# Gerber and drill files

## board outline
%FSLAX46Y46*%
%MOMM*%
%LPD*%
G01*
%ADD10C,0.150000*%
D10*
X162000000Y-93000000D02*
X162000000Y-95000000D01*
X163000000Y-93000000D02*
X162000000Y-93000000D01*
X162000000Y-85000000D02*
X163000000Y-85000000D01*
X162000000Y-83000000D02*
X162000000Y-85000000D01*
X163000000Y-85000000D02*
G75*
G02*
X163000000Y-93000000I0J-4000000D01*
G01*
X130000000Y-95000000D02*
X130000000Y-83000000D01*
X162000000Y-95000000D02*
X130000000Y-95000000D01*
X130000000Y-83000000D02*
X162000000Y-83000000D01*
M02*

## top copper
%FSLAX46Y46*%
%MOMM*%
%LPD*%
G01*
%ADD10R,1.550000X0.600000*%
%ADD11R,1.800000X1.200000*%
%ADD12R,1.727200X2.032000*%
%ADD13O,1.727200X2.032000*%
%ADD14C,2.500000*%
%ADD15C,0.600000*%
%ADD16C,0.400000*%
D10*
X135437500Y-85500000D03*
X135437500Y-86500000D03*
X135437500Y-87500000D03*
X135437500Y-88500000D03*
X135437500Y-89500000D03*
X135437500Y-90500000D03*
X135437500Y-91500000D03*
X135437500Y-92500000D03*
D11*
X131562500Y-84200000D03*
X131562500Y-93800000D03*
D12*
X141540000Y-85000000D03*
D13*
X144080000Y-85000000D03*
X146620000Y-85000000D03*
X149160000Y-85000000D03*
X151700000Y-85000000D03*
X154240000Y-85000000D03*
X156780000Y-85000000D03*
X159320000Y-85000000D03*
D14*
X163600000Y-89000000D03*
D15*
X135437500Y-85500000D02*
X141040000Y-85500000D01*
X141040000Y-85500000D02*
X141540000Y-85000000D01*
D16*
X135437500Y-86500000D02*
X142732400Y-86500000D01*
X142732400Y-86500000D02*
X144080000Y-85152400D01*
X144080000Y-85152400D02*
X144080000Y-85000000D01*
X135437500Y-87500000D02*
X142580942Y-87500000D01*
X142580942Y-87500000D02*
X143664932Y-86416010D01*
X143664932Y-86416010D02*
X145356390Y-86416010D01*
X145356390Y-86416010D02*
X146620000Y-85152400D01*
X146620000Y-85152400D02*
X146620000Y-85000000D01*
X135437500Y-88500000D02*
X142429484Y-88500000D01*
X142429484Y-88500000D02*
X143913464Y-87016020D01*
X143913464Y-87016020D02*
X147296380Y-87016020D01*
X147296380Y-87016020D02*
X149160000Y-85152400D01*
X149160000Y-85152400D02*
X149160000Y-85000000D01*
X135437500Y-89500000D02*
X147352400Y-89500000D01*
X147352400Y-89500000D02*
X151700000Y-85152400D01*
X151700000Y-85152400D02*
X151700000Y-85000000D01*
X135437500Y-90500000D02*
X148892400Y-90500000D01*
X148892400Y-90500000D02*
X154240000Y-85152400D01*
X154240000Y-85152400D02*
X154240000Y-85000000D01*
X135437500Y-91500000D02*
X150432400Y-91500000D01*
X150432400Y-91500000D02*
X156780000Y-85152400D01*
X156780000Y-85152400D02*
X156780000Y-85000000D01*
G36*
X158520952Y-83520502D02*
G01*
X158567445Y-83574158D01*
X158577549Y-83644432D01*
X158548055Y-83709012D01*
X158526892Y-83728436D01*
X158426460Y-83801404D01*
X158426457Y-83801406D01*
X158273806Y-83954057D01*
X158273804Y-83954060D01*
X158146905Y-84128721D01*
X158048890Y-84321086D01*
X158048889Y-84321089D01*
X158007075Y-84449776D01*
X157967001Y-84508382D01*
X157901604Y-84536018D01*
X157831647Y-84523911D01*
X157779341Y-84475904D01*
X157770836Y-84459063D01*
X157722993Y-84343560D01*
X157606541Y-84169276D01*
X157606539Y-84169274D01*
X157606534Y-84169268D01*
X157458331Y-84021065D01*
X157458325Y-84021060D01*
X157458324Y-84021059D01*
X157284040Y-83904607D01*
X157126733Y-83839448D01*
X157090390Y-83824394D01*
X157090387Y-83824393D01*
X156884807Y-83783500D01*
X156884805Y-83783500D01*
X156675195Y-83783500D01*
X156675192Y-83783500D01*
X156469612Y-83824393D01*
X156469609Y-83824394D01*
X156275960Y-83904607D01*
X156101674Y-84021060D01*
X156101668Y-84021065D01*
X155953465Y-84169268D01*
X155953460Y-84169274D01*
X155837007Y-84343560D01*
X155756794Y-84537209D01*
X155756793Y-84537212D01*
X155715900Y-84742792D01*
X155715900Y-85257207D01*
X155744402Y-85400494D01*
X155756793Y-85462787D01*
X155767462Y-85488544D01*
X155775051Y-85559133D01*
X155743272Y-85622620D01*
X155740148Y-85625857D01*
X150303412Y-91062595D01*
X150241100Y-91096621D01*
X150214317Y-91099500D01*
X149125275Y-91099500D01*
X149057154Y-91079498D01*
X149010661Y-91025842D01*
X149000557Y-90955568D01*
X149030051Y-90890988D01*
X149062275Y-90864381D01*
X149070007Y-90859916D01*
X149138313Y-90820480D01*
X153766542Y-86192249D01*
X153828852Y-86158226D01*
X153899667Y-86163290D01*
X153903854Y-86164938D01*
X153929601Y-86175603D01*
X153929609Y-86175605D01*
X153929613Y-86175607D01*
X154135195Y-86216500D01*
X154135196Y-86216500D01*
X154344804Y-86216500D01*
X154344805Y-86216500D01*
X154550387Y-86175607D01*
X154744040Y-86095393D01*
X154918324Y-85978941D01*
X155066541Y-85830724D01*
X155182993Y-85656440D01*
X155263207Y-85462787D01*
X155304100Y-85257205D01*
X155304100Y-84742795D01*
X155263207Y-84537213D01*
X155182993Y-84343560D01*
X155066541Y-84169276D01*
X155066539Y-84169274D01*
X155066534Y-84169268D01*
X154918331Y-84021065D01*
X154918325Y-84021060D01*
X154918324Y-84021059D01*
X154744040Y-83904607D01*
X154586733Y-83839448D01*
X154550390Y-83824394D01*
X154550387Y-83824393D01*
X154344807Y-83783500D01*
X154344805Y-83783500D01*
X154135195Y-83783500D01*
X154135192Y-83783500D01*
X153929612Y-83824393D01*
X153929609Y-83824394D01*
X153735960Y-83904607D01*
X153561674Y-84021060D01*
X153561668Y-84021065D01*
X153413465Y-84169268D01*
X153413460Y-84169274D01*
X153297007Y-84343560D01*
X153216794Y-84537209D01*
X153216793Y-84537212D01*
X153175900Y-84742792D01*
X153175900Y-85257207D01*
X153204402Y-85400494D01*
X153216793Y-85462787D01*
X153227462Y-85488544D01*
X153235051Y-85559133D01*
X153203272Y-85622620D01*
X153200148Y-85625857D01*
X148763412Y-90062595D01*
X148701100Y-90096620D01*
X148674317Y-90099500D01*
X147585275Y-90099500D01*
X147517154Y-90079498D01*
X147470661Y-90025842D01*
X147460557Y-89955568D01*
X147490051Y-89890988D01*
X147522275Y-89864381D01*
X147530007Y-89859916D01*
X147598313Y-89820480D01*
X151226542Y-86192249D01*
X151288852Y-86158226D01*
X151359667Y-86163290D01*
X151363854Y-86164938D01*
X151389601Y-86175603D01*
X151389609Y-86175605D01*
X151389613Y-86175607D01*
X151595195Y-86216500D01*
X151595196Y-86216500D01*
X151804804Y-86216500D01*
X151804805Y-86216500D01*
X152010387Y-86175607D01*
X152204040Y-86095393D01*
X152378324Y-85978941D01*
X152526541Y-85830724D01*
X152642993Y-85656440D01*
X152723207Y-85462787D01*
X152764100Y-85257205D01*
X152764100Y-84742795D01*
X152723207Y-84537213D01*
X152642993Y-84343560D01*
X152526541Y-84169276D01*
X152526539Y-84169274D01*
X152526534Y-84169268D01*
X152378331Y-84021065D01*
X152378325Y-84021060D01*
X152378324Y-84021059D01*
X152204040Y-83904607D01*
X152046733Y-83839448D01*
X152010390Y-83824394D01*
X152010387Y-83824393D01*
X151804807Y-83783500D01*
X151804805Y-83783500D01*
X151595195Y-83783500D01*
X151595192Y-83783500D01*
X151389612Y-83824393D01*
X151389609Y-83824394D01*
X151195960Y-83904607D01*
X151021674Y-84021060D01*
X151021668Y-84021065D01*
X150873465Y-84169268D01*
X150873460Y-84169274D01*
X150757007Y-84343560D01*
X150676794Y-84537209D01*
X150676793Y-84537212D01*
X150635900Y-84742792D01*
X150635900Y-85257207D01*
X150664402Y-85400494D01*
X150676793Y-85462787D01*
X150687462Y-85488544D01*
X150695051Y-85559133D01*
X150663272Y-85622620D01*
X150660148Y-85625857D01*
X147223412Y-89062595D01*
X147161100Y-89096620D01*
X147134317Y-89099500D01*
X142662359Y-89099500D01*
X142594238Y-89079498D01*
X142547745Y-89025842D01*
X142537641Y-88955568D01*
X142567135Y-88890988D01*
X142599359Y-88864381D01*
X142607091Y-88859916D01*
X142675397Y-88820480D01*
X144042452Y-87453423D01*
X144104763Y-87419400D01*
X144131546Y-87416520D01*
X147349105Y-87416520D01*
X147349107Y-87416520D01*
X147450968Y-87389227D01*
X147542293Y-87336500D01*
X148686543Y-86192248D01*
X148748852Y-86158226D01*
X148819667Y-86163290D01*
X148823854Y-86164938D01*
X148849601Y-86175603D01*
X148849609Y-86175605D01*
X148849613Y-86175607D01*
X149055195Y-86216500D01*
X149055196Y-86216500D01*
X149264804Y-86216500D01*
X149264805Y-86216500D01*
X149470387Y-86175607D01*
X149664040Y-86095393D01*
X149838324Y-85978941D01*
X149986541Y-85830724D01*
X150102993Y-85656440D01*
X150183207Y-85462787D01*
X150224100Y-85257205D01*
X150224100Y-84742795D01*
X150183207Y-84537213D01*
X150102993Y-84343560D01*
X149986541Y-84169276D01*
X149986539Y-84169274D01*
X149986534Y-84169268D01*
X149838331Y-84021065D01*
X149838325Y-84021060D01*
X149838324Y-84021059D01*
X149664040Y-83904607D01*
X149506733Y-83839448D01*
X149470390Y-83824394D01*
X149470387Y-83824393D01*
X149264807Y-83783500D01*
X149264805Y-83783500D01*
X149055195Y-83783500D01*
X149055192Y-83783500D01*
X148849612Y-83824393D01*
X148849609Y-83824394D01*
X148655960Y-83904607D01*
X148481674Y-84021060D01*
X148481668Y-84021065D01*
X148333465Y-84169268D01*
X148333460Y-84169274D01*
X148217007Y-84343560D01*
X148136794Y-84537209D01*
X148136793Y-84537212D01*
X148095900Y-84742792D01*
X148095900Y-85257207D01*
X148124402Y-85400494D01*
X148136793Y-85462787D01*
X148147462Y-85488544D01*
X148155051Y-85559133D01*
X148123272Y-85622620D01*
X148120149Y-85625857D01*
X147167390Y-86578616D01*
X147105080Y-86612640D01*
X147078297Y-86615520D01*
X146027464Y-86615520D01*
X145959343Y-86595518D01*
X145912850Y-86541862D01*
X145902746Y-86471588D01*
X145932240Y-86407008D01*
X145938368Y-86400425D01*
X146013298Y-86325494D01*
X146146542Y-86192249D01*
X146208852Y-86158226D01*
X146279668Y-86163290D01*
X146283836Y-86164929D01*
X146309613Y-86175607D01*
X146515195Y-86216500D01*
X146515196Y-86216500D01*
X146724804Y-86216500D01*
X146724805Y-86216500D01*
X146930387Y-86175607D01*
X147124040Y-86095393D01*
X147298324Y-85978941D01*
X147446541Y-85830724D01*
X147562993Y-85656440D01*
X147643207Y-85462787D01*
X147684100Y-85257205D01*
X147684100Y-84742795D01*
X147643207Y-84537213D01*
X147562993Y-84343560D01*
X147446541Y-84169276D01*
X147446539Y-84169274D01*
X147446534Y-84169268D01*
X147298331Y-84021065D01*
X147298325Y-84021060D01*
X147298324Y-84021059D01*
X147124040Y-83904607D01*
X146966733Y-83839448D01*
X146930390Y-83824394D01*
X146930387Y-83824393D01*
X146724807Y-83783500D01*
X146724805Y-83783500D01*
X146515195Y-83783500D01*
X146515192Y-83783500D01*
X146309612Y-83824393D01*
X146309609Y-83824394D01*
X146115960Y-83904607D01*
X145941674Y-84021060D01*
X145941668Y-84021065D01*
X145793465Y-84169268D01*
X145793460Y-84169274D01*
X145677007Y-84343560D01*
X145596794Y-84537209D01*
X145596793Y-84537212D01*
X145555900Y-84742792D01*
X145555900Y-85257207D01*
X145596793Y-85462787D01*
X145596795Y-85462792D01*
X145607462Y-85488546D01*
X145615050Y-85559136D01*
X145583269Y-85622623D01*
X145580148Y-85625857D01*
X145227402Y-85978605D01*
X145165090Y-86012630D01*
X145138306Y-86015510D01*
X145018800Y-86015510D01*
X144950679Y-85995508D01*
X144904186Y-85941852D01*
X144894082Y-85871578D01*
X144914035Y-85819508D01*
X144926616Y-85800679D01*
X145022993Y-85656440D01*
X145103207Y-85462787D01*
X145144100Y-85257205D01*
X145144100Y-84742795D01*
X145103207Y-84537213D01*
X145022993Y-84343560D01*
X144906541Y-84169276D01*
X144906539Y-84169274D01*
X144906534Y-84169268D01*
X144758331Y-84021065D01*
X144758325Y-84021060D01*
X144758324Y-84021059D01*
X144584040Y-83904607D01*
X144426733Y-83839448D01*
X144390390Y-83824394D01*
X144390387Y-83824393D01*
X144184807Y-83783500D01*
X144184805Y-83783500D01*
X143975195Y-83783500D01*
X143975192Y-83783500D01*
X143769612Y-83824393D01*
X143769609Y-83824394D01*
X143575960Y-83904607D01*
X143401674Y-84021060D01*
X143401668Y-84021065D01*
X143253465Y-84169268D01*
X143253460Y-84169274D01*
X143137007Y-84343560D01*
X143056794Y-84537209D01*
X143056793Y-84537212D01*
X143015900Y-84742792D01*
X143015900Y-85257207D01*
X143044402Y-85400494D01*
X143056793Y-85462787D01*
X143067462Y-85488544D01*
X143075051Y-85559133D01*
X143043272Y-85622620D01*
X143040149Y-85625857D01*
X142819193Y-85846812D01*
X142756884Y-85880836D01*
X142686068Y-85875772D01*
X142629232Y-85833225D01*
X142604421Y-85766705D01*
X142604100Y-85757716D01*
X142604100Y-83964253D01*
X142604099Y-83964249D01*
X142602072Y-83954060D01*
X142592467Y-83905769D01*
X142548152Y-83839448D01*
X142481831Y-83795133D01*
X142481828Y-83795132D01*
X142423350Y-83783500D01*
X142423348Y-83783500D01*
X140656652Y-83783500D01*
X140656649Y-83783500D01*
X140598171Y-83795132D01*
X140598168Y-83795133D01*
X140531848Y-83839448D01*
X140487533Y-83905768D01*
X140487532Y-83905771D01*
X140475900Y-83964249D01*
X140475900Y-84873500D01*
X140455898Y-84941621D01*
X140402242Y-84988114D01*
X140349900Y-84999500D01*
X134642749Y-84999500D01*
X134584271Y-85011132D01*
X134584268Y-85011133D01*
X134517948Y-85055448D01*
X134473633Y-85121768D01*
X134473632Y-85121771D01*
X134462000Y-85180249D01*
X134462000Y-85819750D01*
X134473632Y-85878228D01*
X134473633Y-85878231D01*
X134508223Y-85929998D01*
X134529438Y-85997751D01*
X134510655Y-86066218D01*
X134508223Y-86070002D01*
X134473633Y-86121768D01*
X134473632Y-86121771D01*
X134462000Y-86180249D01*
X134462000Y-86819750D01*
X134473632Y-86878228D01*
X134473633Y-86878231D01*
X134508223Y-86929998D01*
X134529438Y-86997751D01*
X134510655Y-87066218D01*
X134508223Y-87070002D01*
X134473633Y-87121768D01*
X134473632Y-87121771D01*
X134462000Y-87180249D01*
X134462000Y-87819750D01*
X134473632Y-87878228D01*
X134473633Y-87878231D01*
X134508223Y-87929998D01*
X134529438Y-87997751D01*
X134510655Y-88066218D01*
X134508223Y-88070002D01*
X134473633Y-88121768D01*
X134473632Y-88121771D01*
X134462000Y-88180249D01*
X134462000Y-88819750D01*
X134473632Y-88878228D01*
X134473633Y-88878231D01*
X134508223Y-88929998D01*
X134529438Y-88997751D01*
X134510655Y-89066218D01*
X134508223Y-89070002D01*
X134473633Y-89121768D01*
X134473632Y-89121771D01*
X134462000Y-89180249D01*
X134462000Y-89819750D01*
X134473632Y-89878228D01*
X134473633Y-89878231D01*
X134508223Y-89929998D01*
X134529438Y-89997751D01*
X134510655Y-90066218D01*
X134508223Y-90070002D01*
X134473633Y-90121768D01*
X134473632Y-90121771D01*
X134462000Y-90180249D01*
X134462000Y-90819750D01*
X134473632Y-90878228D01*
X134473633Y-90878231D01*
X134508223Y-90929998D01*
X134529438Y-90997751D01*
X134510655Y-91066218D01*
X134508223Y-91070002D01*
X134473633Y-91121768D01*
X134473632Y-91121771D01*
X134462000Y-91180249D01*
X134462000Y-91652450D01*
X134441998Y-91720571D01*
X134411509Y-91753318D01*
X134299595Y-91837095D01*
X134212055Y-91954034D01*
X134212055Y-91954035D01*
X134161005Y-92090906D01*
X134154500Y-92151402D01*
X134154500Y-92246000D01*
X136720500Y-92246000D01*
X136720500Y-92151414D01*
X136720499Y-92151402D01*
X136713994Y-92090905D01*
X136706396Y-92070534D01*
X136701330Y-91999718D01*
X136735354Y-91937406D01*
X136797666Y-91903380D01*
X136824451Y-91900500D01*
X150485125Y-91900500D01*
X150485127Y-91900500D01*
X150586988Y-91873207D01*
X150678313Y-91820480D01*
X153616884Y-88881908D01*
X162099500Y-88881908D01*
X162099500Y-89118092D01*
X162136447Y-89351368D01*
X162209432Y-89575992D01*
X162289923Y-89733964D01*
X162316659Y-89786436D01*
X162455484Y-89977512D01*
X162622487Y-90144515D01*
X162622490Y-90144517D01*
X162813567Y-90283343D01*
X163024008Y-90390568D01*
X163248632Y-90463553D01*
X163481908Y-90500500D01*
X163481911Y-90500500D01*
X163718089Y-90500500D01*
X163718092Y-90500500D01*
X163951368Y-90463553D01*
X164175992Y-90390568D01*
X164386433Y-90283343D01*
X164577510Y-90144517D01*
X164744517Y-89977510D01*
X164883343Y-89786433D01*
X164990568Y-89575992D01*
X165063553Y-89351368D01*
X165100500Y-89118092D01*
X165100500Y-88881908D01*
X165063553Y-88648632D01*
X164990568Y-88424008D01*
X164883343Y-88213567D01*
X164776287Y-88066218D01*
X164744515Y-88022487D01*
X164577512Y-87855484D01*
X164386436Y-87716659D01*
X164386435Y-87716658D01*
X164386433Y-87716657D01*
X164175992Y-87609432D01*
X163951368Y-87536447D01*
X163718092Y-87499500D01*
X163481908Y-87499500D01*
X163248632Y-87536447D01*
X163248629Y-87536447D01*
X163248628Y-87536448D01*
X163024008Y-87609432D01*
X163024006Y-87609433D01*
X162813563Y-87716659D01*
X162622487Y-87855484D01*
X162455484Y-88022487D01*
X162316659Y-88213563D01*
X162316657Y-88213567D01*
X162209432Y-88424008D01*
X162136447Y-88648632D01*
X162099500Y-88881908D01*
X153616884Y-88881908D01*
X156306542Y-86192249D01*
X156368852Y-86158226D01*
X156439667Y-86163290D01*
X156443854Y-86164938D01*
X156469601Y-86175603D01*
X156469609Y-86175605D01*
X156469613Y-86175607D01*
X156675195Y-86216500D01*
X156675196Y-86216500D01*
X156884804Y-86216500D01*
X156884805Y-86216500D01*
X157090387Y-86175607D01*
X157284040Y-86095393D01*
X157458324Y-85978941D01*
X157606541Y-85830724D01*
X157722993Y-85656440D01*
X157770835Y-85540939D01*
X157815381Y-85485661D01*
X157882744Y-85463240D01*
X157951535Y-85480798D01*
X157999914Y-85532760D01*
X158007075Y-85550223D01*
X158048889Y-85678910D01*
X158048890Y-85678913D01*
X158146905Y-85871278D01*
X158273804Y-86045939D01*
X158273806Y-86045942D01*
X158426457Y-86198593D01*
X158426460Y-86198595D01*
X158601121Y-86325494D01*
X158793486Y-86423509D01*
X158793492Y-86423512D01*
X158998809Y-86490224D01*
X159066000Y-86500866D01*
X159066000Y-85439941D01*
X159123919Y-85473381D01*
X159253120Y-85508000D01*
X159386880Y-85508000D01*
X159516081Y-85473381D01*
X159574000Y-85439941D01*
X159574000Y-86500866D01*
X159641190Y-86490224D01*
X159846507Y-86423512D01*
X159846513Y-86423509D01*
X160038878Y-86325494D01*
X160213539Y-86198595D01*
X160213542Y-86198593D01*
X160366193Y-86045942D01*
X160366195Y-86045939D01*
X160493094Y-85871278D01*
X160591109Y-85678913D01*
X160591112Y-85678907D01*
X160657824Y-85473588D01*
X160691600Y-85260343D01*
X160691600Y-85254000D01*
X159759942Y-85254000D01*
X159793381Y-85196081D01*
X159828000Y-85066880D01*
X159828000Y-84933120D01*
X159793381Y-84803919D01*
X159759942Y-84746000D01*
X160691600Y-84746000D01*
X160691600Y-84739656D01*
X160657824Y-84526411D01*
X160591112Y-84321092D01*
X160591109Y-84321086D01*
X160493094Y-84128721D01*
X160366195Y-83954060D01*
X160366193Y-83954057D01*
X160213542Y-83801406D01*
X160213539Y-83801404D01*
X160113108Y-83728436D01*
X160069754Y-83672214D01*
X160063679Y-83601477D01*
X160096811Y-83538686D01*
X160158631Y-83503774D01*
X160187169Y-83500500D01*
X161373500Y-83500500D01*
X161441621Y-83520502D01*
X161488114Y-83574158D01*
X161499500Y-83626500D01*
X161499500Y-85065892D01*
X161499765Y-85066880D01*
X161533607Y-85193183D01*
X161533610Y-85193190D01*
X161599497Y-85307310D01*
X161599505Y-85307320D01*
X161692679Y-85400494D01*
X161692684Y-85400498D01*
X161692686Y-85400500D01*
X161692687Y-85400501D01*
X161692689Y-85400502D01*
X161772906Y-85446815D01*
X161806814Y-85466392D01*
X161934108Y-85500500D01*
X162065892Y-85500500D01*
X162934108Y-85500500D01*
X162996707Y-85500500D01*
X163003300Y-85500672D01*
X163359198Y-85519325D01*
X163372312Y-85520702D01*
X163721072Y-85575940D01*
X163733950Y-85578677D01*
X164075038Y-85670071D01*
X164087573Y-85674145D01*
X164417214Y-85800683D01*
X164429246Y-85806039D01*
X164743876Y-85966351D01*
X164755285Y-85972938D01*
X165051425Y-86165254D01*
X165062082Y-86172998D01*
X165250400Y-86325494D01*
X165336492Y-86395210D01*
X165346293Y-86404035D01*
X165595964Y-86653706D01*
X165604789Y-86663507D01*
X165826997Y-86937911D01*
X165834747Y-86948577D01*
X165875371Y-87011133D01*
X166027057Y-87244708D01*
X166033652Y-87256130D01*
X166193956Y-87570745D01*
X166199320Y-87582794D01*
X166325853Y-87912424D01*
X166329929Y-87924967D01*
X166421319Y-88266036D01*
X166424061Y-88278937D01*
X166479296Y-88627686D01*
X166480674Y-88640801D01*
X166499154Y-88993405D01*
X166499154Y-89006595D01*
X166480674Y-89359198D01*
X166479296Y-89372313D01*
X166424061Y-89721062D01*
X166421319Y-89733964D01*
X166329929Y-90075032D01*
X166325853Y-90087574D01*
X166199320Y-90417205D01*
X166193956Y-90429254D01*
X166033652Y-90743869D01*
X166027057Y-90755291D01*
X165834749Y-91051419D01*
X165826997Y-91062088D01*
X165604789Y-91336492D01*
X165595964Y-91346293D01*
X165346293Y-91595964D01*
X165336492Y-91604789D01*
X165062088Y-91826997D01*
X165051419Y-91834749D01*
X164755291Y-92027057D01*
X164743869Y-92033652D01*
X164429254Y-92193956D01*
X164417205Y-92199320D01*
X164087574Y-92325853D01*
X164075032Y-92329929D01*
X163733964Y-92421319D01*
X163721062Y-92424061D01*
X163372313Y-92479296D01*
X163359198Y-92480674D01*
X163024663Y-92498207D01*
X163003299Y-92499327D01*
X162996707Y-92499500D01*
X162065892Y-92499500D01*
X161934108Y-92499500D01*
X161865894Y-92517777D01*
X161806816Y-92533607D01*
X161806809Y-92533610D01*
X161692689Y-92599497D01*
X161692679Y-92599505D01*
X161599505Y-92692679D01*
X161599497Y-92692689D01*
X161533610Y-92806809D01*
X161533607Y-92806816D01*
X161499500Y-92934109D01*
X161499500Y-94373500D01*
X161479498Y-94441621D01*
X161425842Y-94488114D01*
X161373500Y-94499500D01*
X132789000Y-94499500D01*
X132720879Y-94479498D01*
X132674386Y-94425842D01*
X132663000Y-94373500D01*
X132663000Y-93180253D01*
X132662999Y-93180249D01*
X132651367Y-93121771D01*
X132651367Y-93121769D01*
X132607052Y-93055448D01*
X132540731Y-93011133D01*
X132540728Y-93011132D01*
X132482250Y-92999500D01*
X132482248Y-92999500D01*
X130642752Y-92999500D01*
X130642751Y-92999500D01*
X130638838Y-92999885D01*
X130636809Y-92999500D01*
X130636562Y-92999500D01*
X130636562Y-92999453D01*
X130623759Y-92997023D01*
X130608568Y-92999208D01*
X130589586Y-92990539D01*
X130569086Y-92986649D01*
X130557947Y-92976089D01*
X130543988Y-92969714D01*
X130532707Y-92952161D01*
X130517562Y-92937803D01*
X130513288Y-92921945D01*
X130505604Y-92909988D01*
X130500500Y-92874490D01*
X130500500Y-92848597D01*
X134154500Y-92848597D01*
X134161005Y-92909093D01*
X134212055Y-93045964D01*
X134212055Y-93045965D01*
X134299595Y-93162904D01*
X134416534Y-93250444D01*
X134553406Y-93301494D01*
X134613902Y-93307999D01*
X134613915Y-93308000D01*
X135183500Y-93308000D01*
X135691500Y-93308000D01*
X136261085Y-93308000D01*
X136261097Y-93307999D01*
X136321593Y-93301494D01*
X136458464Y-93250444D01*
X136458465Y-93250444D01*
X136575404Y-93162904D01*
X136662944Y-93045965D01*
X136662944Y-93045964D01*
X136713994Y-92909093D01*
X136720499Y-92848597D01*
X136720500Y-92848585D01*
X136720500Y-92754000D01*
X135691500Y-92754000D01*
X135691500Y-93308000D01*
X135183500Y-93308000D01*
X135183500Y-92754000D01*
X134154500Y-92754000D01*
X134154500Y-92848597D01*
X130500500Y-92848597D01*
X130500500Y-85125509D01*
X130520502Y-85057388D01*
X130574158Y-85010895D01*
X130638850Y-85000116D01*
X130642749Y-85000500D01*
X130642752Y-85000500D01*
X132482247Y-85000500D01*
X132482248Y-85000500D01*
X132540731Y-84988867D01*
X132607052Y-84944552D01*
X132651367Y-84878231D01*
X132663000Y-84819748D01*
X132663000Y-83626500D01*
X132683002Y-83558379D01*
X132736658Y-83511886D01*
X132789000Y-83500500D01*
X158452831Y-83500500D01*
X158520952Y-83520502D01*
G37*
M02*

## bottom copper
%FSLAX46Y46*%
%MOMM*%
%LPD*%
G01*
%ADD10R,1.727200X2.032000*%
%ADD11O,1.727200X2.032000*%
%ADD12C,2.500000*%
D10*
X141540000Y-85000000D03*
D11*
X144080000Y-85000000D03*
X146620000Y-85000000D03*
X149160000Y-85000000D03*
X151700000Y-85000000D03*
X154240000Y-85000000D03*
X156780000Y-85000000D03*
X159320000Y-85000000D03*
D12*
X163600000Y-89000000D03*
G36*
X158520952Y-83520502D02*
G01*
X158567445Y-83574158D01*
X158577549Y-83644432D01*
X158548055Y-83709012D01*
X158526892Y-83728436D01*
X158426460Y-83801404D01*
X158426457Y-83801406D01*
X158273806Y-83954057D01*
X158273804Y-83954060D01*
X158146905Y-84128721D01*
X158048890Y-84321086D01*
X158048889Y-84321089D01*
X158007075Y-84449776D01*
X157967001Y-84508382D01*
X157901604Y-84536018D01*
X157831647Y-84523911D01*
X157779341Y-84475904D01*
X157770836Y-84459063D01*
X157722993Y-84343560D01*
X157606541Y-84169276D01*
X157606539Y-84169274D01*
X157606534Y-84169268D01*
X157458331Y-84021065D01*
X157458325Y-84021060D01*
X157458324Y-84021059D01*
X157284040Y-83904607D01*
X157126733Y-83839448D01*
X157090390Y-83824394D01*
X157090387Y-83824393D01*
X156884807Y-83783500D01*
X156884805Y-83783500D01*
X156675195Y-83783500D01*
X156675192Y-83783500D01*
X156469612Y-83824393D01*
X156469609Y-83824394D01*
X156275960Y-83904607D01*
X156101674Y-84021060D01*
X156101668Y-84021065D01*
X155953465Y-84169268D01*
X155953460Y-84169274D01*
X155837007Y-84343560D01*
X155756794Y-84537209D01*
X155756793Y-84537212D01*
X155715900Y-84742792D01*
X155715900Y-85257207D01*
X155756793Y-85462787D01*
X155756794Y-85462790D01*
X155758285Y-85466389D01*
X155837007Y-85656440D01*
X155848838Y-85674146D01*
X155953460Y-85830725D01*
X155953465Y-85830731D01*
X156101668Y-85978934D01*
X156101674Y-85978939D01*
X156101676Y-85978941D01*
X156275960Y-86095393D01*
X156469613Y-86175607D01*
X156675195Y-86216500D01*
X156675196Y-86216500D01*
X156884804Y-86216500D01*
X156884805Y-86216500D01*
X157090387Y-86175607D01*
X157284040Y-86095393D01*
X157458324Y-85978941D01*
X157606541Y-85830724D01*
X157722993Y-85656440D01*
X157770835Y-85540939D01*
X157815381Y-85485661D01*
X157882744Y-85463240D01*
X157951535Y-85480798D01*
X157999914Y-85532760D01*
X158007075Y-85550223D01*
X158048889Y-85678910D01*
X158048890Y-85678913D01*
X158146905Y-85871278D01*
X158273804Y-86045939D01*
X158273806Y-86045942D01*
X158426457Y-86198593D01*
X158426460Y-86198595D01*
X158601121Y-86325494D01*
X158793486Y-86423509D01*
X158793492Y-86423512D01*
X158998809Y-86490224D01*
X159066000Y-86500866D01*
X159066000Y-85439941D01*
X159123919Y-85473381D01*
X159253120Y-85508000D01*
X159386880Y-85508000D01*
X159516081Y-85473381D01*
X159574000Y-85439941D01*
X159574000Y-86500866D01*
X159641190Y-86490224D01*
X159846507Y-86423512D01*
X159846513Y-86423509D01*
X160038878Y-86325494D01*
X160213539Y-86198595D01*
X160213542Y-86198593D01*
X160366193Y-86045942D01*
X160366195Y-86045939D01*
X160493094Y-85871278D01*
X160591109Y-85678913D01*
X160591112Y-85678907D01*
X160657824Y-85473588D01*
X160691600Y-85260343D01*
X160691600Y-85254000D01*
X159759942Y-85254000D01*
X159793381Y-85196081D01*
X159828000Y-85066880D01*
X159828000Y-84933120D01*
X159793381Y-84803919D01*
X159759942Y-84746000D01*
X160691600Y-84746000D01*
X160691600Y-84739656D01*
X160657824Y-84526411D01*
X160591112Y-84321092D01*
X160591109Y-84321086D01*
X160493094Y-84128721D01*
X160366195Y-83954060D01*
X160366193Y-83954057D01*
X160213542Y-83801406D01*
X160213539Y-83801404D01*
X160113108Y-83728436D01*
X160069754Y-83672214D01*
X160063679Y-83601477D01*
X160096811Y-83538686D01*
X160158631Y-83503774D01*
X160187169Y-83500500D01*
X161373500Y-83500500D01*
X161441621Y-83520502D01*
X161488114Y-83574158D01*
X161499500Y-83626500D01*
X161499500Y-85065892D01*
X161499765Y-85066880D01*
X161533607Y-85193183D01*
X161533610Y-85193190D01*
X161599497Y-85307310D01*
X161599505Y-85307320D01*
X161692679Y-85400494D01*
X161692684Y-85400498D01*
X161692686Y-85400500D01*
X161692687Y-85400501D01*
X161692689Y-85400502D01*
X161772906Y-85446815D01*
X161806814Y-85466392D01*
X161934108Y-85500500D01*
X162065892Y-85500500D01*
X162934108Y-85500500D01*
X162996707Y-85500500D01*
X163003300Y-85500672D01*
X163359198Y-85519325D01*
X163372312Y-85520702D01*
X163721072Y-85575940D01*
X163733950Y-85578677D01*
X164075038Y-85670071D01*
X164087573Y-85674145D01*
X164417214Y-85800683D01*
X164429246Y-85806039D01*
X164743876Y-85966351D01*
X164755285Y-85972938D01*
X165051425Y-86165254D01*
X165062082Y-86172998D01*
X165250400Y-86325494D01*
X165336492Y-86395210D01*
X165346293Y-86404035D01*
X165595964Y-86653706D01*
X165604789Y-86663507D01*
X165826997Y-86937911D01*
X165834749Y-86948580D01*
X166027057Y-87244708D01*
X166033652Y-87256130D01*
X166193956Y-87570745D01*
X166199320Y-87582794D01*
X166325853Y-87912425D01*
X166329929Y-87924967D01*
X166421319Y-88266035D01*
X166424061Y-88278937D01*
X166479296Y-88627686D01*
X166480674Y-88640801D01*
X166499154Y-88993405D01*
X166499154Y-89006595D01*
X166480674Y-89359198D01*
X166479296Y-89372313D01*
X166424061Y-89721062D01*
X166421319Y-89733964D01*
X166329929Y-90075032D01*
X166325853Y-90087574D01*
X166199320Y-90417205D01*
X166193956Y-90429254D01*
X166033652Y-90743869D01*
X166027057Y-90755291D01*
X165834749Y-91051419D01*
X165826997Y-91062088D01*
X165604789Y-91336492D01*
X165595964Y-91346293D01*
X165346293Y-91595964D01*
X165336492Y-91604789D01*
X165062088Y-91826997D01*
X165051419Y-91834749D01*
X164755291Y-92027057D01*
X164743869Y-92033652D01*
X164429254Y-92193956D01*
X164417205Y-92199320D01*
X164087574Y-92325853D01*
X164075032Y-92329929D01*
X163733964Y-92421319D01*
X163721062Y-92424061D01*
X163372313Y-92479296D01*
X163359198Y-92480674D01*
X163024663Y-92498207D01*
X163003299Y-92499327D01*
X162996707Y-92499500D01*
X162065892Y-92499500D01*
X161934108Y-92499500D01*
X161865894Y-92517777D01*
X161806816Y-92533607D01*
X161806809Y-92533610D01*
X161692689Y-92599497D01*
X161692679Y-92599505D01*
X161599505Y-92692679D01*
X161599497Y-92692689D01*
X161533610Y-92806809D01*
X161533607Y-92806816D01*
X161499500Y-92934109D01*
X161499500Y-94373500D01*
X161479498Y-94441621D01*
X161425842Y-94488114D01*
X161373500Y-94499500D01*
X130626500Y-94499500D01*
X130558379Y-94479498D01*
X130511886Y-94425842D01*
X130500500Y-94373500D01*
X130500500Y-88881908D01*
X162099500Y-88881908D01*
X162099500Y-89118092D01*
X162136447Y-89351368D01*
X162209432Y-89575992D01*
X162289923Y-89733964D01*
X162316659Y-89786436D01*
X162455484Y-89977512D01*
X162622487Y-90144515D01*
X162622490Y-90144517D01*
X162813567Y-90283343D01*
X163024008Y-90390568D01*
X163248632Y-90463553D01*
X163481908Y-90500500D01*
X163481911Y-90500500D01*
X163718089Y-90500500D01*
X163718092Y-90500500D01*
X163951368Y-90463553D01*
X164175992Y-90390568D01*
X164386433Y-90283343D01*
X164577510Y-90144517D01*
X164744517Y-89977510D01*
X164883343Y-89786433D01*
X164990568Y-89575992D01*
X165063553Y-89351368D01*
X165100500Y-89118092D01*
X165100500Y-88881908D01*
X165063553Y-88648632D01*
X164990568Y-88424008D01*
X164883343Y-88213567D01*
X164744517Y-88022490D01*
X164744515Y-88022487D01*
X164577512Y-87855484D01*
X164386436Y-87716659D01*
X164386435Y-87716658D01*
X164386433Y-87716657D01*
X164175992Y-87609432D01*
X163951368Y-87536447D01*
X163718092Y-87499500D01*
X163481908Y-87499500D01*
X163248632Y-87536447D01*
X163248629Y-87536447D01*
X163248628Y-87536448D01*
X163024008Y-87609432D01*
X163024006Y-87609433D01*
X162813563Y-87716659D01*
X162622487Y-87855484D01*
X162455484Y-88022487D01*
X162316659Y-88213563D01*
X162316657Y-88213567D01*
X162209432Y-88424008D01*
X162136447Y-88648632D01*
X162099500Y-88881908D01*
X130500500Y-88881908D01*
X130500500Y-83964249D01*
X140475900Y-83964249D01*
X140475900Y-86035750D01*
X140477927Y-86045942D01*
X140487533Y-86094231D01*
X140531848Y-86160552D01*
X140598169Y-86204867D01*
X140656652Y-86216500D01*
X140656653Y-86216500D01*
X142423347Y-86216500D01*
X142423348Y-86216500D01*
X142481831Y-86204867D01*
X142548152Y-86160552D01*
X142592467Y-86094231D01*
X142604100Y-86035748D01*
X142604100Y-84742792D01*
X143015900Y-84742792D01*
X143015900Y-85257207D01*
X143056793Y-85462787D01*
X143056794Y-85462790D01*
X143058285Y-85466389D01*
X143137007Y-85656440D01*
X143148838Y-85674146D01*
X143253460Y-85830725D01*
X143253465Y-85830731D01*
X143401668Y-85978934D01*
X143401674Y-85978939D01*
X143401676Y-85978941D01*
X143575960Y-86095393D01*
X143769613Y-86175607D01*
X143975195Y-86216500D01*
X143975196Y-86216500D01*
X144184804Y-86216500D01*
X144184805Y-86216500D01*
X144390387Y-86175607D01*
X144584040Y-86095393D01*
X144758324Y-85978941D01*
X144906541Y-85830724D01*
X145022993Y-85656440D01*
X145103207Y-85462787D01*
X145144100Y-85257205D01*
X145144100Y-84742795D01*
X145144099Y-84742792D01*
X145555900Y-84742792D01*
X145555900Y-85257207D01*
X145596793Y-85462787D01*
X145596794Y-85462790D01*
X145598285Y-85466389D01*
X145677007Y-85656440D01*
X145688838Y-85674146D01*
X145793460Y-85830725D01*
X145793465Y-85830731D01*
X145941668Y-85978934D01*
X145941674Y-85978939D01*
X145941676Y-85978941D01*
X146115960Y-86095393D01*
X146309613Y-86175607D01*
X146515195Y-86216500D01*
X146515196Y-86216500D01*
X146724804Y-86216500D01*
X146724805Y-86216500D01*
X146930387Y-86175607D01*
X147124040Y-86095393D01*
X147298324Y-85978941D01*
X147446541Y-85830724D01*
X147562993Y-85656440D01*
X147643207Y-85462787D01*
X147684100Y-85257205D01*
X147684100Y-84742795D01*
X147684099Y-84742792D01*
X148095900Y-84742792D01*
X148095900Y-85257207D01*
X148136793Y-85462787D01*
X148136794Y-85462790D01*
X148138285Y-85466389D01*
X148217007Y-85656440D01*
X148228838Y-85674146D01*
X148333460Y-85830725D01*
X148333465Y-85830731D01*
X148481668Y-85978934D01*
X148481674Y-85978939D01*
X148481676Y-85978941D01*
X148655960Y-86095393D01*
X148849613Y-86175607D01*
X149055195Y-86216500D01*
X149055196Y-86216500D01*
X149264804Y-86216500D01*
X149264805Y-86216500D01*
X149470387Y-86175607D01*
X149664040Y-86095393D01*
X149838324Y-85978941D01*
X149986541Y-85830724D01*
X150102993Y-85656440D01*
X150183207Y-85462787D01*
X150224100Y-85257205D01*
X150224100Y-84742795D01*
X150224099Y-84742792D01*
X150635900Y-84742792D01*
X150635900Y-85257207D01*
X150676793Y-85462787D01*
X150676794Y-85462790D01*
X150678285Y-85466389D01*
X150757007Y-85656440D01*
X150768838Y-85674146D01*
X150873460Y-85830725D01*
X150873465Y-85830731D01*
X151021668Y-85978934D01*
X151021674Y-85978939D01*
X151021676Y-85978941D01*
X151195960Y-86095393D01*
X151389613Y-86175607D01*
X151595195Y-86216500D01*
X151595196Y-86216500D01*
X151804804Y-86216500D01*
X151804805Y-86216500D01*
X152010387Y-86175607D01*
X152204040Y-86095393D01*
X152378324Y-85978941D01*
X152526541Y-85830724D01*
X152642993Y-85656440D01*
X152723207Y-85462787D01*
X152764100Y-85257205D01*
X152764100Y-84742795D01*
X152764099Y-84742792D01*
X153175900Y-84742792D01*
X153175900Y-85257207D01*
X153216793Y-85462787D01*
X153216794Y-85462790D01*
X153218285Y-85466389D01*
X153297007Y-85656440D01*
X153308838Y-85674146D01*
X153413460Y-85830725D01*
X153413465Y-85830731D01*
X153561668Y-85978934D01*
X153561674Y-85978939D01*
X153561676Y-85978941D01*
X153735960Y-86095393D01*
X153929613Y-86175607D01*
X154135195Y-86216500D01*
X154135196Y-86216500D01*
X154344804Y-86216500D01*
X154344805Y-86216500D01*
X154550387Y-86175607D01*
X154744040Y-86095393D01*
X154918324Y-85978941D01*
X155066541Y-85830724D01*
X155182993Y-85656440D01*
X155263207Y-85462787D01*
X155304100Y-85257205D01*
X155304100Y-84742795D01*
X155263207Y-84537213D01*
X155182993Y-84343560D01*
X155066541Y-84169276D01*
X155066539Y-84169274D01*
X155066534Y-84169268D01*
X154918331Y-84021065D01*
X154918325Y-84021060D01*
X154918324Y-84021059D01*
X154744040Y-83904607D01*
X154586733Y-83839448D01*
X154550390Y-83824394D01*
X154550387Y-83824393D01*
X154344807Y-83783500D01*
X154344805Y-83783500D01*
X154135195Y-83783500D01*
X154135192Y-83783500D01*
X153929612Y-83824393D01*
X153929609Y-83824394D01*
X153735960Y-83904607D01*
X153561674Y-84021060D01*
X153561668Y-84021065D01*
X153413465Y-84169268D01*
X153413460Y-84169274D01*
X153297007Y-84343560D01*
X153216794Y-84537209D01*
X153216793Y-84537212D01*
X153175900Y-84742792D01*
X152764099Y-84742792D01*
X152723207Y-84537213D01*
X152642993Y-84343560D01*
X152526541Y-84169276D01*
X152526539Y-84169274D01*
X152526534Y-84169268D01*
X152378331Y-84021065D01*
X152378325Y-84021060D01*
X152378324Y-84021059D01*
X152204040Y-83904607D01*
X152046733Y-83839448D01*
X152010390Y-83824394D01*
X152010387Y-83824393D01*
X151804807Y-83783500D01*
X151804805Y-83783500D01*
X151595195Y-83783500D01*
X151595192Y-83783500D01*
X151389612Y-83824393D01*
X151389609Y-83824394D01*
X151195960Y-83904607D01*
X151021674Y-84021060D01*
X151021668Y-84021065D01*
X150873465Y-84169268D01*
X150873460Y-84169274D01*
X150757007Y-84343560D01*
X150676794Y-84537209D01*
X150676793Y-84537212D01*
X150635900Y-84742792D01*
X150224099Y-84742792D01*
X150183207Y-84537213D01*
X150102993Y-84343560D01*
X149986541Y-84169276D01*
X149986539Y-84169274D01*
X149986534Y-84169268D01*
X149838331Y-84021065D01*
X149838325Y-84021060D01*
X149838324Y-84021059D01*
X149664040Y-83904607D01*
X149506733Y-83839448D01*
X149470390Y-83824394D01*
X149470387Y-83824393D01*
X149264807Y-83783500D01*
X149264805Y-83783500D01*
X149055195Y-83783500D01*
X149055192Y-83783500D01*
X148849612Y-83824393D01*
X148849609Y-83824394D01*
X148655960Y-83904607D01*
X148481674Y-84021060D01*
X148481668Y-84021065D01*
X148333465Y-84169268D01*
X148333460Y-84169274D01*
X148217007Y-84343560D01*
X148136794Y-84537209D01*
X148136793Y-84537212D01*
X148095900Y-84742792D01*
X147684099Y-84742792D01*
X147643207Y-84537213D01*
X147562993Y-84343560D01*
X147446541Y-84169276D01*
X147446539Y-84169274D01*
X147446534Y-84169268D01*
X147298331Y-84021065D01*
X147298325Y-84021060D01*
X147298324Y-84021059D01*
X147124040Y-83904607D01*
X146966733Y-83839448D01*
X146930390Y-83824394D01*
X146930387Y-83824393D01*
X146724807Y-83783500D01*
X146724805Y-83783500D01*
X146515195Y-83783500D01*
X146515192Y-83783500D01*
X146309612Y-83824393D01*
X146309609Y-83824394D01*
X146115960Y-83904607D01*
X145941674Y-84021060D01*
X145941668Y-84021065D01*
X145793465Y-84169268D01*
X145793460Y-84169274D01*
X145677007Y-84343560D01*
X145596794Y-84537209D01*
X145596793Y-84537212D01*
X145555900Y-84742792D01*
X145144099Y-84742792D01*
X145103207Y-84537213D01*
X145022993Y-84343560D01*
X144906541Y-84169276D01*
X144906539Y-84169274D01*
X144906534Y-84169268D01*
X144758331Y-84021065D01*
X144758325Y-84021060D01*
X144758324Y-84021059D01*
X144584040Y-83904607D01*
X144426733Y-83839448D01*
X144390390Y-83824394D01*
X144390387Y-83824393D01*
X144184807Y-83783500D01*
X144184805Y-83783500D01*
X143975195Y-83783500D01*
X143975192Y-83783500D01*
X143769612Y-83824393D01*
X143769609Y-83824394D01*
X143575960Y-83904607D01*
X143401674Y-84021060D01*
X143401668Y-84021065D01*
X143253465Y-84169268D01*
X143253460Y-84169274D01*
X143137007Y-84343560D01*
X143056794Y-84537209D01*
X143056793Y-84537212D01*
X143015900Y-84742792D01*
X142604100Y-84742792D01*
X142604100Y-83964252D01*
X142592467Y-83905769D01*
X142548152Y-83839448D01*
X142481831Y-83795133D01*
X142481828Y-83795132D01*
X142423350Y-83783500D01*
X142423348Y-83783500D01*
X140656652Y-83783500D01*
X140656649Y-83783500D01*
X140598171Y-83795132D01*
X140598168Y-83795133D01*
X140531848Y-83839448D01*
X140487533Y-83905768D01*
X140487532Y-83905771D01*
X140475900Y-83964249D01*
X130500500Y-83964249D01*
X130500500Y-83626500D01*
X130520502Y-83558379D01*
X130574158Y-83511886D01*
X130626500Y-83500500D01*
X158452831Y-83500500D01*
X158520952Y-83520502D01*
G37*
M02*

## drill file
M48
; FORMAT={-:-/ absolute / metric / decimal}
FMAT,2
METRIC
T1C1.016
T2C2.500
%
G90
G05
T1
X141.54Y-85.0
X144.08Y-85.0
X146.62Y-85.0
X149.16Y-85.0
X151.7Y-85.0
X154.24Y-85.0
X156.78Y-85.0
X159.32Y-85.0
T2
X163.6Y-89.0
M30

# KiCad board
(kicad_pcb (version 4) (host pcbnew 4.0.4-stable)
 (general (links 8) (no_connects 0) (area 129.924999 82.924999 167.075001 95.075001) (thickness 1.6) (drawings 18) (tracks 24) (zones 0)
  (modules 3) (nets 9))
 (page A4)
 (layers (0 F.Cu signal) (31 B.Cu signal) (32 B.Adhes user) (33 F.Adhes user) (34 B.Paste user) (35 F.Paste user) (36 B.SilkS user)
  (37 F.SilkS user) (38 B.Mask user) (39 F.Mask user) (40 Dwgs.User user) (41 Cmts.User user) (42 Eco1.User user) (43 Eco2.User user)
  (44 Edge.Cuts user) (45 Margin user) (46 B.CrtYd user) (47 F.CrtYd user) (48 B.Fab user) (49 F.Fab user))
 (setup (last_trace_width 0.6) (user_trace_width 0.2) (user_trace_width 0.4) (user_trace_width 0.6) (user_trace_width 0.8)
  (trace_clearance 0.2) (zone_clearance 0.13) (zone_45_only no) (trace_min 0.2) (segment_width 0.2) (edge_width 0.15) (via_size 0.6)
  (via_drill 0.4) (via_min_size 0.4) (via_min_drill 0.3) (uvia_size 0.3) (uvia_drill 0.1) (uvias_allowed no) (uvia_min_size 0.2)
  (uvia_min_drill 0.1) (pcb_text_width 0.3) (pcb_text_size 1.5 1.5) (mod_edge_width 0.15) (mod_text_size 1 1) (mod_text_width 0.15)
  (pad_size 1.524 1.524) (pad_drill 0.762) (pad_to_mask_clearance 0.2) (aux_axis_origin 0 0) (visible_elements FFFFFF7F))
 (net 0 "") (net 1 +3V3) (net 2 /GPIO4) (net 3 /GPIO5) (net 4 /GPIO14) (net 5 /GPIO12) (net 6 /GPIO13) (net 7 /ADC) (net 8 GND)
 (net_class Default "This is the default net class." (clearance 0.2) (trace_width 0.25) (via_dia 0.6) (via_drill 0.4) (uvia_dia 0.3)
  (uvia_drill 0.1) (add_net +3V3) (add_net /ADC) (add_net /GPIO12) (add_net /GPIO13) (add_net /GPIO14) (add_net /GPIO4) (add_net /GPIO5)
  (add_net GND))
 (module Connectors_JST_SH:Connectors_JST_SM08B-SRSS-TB (layer F.Cu) (at 133.5 89 270)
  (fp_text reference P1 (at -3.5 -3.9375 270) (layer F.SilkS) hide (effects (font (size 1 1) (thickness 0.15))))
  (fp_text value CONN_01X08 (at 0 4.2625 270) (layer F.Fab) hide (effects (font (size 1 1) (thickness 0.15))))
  (pad 1 smd rect (at -3.5 -1.9375 270) (size 0.6 1.55) (layers F.Cu F.Paste F.Mask) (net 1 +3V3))
  (pad 2 smd rect (at -2.5 -1.9375 270) (size 0.6 1.55) (layers F.Cu F.Paste F.Mask) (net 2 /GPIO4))
  (pad 3 smd rect (at -1.5 -1.9375 270) (size 0.6 1.55) (layers F.Cu F.Paste F.Mask) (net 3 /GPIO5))
  (pad 4 smd rect (at -0.5 -1.9375 270) (size 0.6 1.55) (layers F.Cu F.Paste F.Mask) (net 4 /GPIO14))
  (pad 5 smd rect (at 0.5 -1.9375 270) (size 0.6 1.55) (layers F.Cu F.Paste F.Mask) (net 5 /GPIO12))
  (pad 6 smd rect (at 1.5 -1.9375 270) (size 0.6 1.55) (layers F.Cu F.Paste F.Mask) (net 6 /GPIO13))
  (pad 7 smd rect (at 2.5 -1.9375 270) (size 0.6 1.55) (layers F.Cu F.Paste F.Mask) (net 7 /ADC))
  (pad 8 smd rect (at 3.5 -1.9375 270) (size 0.6 1.55) (layers F.Cu F.Paste F.Mask) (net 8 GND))
  (pad "" smd rect (at -4.8 1.9375 270) (size 1.2 1.8) (layers F.Cu F.Paste F.Mask))
  (pad "" smd rect (at 4.8 1.9375 270) (size 1.2 1.8) (layers F.Cu F.Paste F.Mask)))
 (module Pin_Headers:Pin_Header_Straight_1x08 (layer F.Cu) (at 141.54 85 90)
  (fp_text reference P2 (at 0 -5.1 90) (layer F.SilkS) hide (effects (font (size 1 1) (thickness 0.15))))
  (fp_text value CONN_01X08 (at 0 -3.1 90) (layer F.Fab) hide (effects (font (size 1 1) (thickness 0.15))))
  (pad 1 thru_hole rect (at 0 0 90) (size 2.032 1.7272) (drill 1.016) (layers *.Cu *.Mask F.SilkS) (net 1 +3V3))
  (pad 2 thru_hole oval (at 0 2.54 90) (size 2.032 1.7272) (drill 1.016) (layers *.Cu *.Mask F.SilkS) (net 2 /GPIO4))
  (pad 3 thru_hole oval (at 0 5.08 90) (size 2.032 1.7272) (drill 1.016) (layers *.Cu *.Mask F.SilkS) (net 3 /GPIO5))
  (pad 4 thru_hole oval (at 0 7.62 90) (size 2.032 1.7272) (drill 1.016) (layers *.Cu *.Mask F.SilkS) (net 4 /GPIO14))
  (pad 5 thru_hole oval (at 0 10.16 90) (size 2.032 1.7272) (drill 1.016) (layers *.Cu *.Mask F.SilkS) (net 5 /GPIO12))
  (pad 6 thru_hole oval (at 0 12.7 90) (size 2.032 1.7272) (drill 1.016) (layers *.Cu *.Mask F.SilkS) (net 6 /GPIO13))
  (pad 7 thru_hole oval (at 0 15.24 90) (size 2.032 1.7272) (drill 1.016) (layers *.Cu *.Mask F.SilkS) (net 7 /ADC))
  (pad 8 thru_hole oval (at 0 17.78 90) (size 2.032 1.7272) (drill 1.016) (layers *.Cu *.Mask F.SilkS) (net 8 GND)))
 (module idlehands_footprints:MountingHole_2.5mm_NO (layer F.Cu) (at 163.625 89)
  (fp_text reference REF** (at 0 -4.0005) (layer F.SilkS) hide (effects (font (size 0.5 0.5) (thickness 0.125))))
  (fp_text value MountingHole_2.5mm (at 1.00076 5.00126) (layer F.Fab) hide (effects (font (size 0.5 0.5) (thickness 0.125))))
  (pad 1 thru_hole circle (at -0.025 0) (size 2.5 2.5) (drill 2.5) (layers *.Cu)))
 (gr_line (start 162 93) (end 162 95) (layer Edge.Cuts) (width 0.15))
 (gr_line (start 163 93) (end 162 93) (layer Edge.Cuts) (width 0.15))
 (gr_line (start 162 85) (end 163 85) (layer Edge.Cuts) (width 0.15))
 (gr_line (start 162 83) (end 162 85) (layer Edge.Cuts) (width 0.15))
 (gr_arc (start 163 89) (end 163 85) (angle 180) (layer Edge.Cuts) (width 0.15))
 (gr_line (start 130 95) (end 130 83) (layer Edge.Cuts) (width 0.15))
 (gr_line (start 162 95) (end 130 95) (layer Edge.Cuts) (width 0.15))
 (gr_line (start 130 83) (end 162 83) (layer Edge.Cuts) (width 0.15))
 (segment (start 135.4375 85.5) (end 141.04 85.5) (width 0.6) (layer F.Cu) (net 1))
 (segment (start 141.04 85.5) (end 141.54 85) (width 0.6) (layer F.Cu) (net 1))
 (segment (start 135.4375 86.5) (end 142.7324 86.5) (width 0.4) (layer F.Cu) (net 2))
 (segment (start 142.7324 86.5) (end 144.08 85.1524) (width 0.4) (layer F.Cu) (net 2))
 (segment (start 144.08 85.1524) (end 144.08 85) (width 0.4) (layer F.Cu) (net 2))
 (segment (start 135.4375 87.5) (end 142.580942 87.5) (width 0.4) (layer F.Cu) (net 3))
 (segment (start 142.580942 87.5) (end 143.664932 86.41601) (width 0.4) (layer F.Cu) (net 3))
 (segment (start 143.664932 86.41601) (end 145.35639 86.41601) (width 0.4) (layer F.Cu) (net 3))
 (segment (start 145.35639 86.41601) (end 146.62 85.1524) (width 0.4) (layer F.Cu) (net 3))
 (segment (start 146.62 85.1524) (end 146.62 85) (width 0.4) (layer F.Cu) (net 3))
 (segment (start 135.4375 88.5) (end 142.429484 88.5) (width 0.4) (layer F.Cu) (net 4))
 (segment (start 142.429484 88.5) (end 143.913464 87.01602) (width 0.4) (layer F.Cu) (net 4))
 (segment (start 143.913464 87.01602) (end 147.29638 87.01602) (width 0.4) (layer F.Cu) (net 4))
 (segment (start 147.29638 87.01602) (end 149.16 85.1524) (width 0.4) (layer F.Cu) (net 4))
 (segment (start 149.16 85.1524) (end 149.16 85) (width 0.4) (layer F.Cu) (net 4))
 (segment (start 135.4375 89.5) (end 147.3524 89.5) (width 0.4) (layer F.Cu) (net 5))
 (segment (start 147.3524 89.5) (end 151.7 85.1524) (width 0.4) (layer F.Cu) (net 5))
 (segment (start 151.7 85.1524) (end 151.7 85) (width 0.4) (layer F.Cu) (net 5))
 (segment (start 135.4375 90.5) (end 148.8924 90.5) (width 0.4) (layer F.Cu) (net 6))
 (segment (start 148.8924 90.5) (end 154.24 85.1524) (width 0.4) (layer F.Cu) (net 6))
 (segment (start 154.24 85.1524) (end 154.24 85) (width 0.4) (layer F.Cu) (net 6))
 (segment (start 135.4375 91.5) (end 150.4324 91.5) (width 0.4) (layer F.Cu) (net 7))
 (segment (start 150.4324 91.5) (end 156.78 85.1524) (width 0.4) (layer F.Cu) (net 7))
 (segment (start 156.78 85.1524) (end 156.78 85) (width 0.4) (layer F.Cu) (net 7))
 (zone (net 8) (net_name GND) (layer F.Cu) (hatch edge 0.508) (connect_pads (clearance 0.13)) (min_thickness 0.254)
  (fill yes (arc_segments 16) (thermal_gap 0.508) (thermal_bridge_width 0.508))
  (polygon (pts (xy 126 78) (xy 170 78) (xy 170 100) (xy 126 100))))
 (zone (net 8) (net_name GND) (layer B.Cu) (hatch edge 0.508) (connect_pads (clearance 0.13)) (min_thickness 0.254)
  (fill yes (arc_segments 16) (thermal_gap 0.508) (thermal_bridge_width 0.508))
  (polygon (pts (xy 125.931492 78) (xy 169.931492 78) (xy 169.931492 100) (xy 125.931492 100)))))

